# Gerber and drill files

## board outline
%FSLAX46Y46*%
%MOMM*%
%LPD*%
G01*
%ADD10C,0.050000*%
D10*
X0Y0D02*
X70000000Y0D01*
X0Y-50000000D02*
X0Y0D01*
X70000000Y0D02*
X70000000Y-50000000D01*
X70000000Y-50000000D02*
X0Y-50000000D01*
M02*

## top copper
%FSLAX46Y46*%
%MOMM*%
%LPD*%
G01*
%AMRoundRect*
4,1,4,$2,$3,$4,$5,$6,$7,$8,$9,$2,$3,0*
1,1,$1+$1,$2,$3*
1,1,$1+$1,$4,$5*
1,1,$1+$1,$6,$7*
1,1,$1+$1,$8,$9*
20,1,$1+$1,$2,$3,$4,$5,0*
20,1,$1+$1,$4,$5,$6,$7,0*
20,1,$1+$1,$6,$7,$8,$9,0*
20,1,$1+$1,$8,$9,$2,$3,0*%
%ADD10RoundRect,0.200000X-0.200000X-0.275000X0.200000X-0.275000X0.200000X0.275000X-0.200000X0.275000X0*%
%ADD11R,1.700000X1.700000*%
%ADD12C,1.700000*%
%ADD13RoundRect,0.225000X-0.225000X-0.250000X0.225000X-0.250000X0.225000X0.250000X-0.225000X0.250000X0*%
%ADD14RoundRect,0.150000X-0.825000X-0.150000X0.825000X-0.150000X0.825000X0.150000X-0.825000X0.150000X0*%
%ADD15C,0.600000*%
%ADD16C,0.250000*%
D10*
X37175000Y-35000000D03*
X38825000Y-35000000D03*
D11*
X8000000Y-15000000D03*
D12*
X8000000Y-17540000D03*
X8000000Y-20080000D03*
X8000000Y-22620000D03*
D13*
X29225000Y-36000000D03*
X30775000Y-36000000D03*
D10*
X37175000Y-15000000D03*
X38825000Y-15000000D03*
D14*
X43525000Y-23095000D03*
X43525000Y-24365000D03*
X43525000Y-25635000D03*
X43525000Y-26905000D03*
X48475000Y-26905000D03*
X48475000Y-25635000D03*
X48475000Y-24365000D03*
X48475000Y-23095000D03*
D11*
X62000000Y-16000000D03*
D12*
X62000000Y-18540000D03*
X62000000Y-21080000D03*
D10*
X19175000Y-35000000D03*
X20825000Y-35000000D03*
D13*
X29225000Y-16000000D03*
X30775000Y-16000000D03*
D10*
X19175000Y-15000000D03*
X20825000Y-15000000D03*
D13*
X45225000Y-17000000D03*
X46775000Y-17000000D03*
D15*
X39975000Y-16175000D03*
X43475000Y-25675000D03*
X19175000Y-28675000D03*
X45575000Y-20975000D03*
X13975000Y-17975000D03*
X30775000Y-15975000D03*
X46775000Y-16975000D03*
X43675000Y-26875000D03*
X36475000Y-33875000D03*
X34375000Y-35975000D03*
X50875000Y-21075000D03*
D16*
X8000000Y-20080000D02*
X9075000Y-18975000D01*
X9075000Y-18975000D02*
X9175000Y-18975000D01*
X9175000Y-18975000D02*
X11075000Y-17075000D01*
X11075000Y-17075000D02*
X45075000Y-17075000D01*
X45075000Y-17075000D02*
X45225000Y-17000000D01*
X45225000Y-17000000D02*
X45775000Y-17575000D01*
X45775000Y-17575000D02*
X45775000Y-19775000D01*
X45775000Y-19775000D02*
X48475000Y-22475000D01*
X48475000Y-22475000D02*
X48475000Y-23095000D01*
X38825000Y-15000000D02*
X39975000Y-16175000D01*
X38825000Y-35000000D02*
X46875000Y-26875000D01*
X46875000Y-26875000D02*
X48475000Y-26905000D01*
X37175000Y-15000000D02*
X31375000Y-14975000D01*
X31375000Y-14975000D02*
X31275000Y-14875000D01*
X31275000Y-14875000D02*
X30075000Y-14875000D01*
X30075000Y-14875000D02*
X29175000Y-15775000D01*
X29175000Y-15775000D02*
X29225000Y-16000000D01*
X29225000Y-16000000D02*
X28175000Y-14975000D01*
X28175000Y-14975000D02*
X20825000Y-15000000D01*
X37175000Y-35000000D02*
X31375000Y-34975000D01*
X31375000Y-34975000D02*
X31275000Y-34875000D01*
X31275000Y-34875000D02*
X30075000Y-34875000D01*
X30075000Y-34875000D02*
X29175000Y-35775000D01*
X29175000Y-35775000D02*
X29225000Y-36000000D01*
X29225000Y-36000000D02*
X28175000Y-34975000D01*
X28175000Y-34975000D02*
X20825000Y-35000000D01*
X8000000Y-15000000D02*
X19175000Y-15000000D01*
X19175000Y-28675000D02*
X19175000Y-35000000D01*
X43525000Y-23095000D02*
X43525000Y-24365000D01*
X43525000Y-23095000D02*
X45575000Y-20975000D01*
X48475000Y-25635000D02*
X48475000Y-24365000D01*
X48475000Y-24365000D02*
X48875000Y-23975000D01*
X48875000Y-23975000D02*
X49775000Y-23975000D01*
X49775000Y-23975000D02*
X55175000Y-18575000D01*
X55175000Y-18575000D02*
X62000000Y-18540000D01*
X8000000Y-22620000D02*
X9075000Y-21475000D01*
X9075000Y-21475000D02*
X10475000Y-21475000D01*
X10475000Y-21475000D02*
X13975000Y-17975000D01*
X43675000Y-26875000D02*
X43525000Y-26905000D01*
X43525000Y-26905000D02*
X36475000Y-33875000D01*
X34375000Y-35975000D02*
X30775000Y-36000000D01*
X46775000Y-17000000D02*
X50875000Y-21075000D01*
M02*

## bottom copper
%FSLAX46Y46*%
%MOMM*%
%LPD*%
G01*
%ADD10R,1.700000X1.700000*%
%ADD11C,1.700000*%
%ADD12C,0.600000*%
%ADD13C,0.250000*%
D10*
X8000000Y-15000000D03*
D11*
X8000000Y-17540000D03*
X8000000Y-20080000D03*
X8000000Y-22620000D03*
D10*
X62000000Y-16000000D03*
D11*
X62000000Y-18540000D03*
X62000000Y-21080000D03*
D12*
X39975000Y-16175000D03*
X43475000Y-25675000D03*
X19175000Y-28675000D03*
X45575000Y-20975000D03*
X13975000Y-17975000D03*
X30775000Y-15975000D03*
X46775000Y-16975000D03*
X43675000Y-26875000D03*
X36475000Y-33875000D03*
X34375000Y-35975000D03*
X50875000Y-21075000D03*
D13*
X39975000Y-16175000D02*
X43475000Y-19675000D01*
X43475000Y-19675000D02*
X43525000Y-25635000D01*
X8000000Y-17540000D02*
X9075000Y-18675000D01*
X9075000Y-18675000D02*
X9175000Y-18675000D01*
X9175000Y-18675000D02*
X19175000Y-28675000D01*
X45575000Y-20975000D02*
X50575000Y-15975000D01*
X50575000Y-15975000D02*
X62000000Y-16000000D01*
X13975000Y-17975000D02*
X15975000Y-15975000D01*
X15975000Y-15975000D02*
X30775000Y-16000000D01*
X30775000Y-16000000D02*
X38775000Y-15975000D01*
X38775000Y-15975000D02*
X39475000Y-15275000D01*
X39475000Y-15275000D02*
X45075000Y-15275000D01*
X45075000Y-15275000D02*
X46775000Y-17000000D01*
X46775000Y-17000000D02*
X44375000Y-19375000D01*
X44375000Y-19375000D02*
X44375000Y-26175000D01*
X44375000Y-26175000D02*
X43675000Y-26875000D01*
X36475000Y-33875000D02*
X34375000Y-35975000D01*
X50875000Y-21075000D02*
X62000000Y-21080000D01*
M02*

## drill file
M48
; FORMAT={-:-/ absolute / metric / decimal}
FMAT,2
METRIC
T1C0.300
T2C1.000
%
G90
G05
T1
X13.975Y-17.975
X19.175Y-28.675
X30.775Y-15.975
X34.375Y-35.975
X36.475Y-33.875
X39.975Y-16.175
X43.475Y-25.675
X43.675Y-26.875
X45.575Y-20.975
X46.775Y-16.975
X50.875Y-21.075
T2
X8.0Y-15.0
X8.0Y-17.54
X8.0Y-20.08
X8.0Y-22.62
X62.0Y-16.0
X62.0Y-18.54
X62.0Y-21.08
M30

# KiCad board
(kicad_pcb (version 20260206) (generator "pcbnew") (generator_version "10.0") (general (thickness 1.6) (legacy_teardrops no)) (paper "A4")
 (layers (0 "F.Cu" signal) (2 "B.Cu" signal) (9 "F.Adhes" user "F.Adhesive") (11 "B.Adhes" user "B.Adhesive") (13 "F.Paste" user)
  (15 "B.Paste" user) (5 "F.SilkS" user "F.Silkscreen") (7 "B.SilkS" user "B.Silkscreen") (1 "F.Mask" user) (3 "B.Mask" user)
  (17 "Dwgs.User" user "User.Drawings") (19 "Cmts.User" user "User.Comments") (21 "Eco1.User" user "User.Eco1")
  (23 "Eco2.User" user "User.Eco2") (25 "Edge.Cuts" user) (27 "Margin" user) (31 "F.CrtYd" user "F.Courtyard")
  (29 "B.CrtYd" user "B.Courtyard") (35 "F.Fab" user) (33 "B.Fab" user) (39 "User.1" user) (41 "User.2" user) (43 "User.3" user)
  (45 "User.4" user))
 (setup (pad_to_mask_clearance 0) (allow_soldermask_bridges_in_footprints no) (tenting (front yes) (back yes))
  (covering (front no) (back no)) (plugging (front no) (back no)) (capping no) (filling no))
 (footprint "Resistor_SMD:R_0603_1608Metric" (layer "F.Cu") (at 38 35)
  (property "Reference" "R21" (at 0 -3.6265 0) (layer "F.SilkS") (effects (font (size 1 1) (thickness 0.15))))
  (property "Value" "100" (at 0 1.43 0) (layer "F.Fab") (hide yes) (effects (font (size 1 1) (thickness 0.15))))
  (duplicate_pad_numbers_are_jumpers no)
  (pad "1" smd roundrect (at -0.825 0) (size 0.8 0.95) (layers "F.Cu" "F.Mask" "F.Paste") (roundrect_rratio 0.25) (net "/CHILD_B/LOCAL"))
  (pad "2" smd roundrect (at 0.825 0) (size 0.8 0.95) (layers "F.Cu" "F.Mask" "F.Paste") (roundrect_rratio 0.25) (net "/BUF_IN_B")))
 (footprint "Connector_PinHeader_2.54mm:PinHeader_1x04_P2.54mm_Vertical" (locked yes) (layer "F.Cu") (at 8 15)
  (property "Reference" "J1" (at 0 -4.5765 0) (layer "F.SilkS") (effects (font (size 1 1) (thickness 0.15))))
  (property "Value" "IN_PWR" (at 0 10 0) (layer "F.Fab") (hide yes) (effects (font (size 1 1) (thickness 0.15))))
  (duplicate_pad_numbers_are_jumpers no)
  (pad "1" thru_hole rect (at 0 0) (size 1.7 1.7) (drill 1) (layers "*.Cu" "*.Mask") (remove_unused_layers no) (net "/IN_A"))
  (pad "2" thru_hole circle (at 0 2.54) (size 1.7 1.7) (drill 1) (layers "*.Cu" "*.Mask") (remove_unused_layers no) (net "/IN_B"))
  (pad "3" thru_hole circle (at 0 5.08) (size 1.7 1.7) (drill 1) (layers "*.Cu" "*.Mask") (remove_unused_layers no) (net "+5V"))
  (pad "4" thru_hole circle (at 0 7.62) (size 1.7 1.7) (drill 1) (layers "*.Cu" "*.Mask") (remove_unused_layers no) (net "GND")))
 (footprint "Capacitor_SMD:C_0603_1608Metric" (layer "F.Cu") (at 30 36)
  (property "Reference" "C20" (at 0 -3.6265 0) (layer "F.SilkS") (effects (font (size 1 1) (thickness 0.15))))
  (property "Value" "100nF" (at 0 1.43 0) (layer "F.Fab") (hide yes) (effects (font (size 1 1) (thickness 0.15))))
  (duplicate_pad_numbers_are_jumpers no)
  (pad "1" smd roundrect (at -0.775 0) (size 0.9 0.95) (layers "F.Cu" "F.Mask" "F.Paste") (roundrect_rratio 0.25) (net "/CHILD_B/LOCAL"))
  (pad "2" smd roundrect (at 0.775 0) (size 0.9 0.95) (layers "F.Cu" "F.Mask" "F.Paste") (roundrect_rratio 0.25) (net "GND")))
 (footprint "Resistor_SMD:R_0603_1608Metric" (layer "F.Cu") (at 38 15)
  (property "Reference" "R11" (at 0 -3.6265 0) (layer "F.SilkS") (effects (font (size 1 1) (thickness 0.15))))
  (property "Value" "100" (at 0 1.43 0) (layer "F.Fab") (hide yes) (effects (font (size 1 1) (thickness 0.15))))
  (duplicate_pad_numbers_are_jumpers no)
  (pad "1" smd roundrect (at -0.825 0) (size 0.8 0.95) (layers "F.Cu" "F.Mask" "F.Paste") (roundrect_rratio 0.25) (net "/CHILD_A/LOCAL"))
  (pad "2" smd roundrect (at 0.825 0) (size 0.8 0.95) (layers "F.Cu" "F.Mask" "F.Paste") (roundrect_rratio 0.25) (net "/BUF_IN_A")))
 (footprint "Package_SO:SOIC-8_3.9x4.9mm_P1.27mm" (layer "F.Cu") (at 46 25)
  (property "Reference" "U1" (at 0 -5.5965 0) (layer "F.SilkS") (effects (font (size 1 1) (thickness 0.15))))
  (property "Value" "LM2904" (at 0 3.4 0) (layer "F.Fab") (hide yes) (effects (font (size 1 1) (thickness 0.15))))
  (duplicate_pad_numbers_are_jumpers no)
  (pad "1" smd roundrect (at -2.475 -1.905) (size 1.95 0.6) (layers "F.Cu" "F.Mask" "F.Paste") (roundrect_rratio 0.25) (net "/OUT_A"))
  (pad "2" smd roundrect (at -2.475 -0.635) (size 1.95 0.6) (layers "F.Cu" "F.Mask" "F.Paste") (roundrect_rratio 0.25) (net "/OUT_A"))
  (pad "3" smd roundrect (at -2.475 0.635) (size 1.95 0.6) (layers "F.Cu" "F.Mask" "F.Paste") (roundrect_rratio 0.25) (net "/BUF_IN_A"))
  (pad "4" smd roundrect (at -2.475 1.905) (size 1.95 0.6) (layers "F.Cu" "F.Mask" "F.Paste") (roundrect_rratio 0.25) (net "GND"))
  (pad "5" smd roundrect (at 2.475 1.905) (size 1.95 0.6) (layers "F.Cu" "F.Mask" "F.Paste") (roundrect_rratio 0.25) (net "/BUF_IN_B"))
  (pad "6" smd roundrect (at 2.475 0.635) (size 1.95 0.6) (layers "F.Cu" "F.Mask" "F.Paste") (roundrect_rratio 0.25) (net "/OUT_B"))
  (pad "7" smd roundrect (at 2.475 -0.635) (size 1.95 0.6) (layers "F.Cu" "F.Mask" "F.Paste") (roundrect_rratio 0.25) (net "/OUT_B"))
  (pad "8" smd roundrect (at 2.475 -1.905) (size 1.95 0.6) (layers "F.Cu" "F.Mask" "F.Paste") (roundrect_rratio 0.25) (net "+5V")))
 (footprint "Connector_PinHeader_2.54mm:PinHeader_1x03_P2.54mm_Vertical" (layer "F.Cu") (at 62 16)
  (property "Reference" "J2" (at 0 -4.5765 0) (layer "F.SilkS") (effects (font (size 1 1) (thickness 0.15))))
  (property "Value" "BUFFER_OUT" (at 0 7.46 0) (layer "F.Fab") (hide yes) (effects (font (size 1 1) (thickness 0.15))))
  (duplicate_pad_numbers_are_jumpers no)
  (pad "1" thru_hole rect (at 0 0) (size 1.7 1.7) (drill 1) (layers "*.Cu" "*.Mask") (remove_unused_layers no) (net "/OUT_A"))
  (pad "2" thru_hole circle (at 0 2.54) (size 1.7 1.7) (drill 1) (layers "*.Cu" "*.Mask") (remove_unused_layers no) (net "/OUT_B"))
  (pad "3" thru_hole circle (at 0 5.08) (size 1.7 1.7) (drill 1) (layers "*.Cu" "*.Mask") (remove_unused_layers no) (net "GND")))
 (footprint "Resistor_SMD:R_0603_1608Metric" (layer "F.Cu") (at 20 35)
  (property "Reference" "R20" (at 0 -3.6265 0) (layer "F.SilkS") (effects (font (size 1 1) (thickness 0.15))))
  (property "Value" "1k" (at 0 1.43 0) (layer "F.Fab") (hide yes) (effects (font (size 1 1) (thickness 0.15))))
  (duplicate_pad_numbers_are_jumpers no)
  (pad "1" smd roundrect (at -0.825 0) (size 0.8 0.95) (layers "F.Cu" "F.Mask" "F.Paste") (roundrect_rratio 0.25) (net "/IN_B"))
  (pad "2" smd roundrect (at 0.825 0) (size 0.8 0.95) (layers "F.Cu" "F.Mask" "F.Paste") (roundrect_rratio 0.25) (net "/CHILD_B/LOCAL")))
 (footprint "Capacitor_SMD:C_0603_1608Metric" (layer "F.Cu") (at 30 16)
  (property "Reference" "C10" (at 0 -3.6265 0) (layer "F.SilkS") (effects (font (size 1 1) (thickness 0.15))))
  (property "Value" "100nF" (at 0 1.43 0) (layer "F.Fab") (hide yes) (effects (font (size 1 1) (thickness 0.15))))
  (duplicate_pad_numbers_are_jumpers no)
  (pad "1" smd roundrect (at -0.775 0) (size 0.9 0.95) (layers "F.Cu" "F.Mask" "F.Paste") (roundrect_rratio 0.25) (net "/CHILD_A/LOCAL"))
  (pad "2" smd roundrect (at 0.775 0) (size 0.9 0.95) (layers "F.Cu" "F.Mask" "F.Paste") (roundrect_rratio 0.25) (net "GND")))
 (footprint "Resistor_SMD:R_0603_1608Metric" (layer "F.Cu") (at 20 15)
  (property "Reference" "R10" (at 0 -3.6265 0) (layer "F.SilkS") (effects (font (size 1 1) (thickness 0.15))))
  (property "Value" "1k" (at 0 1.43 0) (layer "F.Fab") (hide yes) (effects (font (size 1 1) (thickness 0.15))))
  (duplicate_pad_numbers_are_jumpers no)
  (pad "1" smd roundrect (at -0.825 0) (size 0.8 0.95) (layers "F.Cu" "F.Mask" "F.Paste") (roundrect_rratio 0.25) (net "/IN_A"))
  (pad "2" smd roundrect (at 0.825 0) (size 0.8 0.95) (layers "F.Cu" "F.Mask" "F.Paste") (roundrect_rratio 0.25) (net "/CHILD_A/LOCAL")))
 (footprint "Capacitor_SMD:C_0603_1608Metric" (layer "F.Cu") (at 46 17)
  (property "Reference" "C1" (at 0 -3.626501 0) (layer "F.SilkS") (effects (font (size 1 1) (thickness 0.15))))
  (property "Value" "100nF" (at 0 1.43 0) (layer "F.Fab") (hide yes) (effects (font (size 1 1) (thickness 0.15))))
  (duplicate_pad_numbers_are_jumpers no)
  (pad "1" smd roundrect (at -0.775 0) (size 0.9 0.95) (layers "F.Cu" "F.Mask" "F.Paste") (roundrect_rratio 0.25) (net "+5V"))
  (pad "2" smd roundrect (at 0.775 0) (size 0.9 0.95) (layers "F.Cu" "F.Mask" "F.Paste") (roundrect_rratio 0.25) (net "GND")))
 (gr_line (start 0 0) (end 70 0) (stroke (width 0.05) (type default)) (layer "Edge.Cuts"))
 (gr_line (start 0 50) (end 0 0) (stroke (width 0.05) (type default)) (layer "Edge.Cuts"))
 (gr_line (start 70 0) (end 70 50) (stroke (width 0.05) (type default)) (layer "Edge.Cuts"))
 (gr_line (start 70 50) (end 0 50) (stroke (width 0.05) (type default)) (layer "Edge.Cuts"))
 (segment (start 8 20.08) (end 9.075 18.975) (width 0.25) (layer "F.Cu") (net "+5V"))
 (segment (start 9.075 18.975) (end 9.175 18.975) (width 0.25) (layer "F.Cu") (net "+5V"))
 (segment (start 9.175 18.975) (end 11.075 17.075) (width 0.25) (layer "F.Cu") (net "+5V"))
 (segment (start 11.075 17.075) (end 45.075 17.075) (width 0.25) (layer "F.Cu") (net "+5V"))
 (segment (start 45.075 17.075) (end 45.225 17) (width 0.25) (layer "F.Cu") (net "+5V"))
 (segment (start 45.225 17) (end 45.775 17.575) (width 0.25) (layer "F.Cu") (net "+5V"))
 (segment (start 45.775 17.575) (end 45.775 19.775) (width 0.25) (layer "F.Cu") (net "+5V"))
 (segment (start 45.775 19.775) (end 48.475 22.475) (width 0.25) (layer "F.Cu") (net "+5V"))
 (segment (start 48.475 22.475) (end 48.475 23.095) (width 0.25) (layer "F.Cu") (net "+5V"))
 (segment (start 38.825 15) (end 39.975 16.175) (width 0.25) (layer "F.Cu") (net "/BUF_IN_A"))
 (via (at 39.975 16.175) (size 0.6) (drill 0.3) (layers "F.Cu" "B.Cu") (capping no) (covering (front no) (back no))
  (plugging (front no) (back no)) (filling no) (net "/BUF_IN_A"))
 (segment (start 39.975 16.175) (end 43.475 19.675) (width 0.25) (layer "B.Cu") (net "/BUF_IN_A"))
 (segment (start 43.475 19.675) (end 43.525 25.635) (width 0.25) (layer "B.Cu") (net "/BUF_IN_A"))
 (via (at 43.475 25.675) (size 0.6) (drill 0.3) (layers "F.Cu" "B.Cu") (capping no) (covering (front no) (back no))
  (plugging (front no) (back no)) (filling no) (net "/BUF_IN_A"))
 (segment (start 38.825 35) (end 46.875 26.875) (width 0.25) (layer "F.Cu") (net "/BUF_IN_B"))
 (segment (start 46.875 26.875) (end 48.475 26.905) (width 0.25) (layer "F.Cu") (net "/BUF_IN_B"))
 (segment (start 37.175 15) (end 31.375 14.975) (width 0.25) (layer "F.Cu") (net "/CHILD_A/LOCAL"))
 (segment (start 31.375 14.975) (end 31.275 14.875) (width 0.25) (layer "F.Cu") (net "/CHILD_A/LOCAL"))
 (segment (start 31.275 14.875) (end 30.075 14.875) (width 0.25) (layer "F.Cu") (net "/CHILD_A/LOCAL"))
 (segment (start 30.075 14.875) (end 29.175 15.775) (width 0.25) (layer "F.Cu") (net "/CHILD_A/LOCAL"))
 (segment (start 29.175 15.775) (end 29.225 16) (width 0.25) (layer "F.Cu") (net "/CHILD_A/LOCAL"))
 (segment (start 29.225 16) (end 28.175 14.975) (width 0.25) (layer "F.Cu") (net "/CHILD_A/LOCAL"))
 (segment (start 28.175 14.975) (end 20.825 15) (width 0.25) (layer "F.Cu") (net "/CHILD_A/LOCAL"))
 (segment (start 37.175 35) (end 31.375 34.975) (width 0.25) (layer "F.Cu") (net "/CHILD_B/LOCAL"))
 (segment (start 31.375 34.975) (end 31.275 34.875) (width 0.25) (layer "F.Cu") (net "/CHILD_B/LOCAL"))
 (segment (start 31.275 34.875) (end 30.075 34.875) (width 0.25) (layer "F.Cu") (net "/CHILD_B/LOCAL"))
 (segment (start 30.075 34.875) (end 29.175 35.775) (width 0.25) (layer "F.Cu") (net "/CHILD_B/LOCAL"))
 (segment (start 29.175 35.775) (end 29.225 36) (width 0.25) (layer "F.Cu") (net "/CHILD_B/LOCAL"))
 (segment (start 29.225 36) (end 28.175 34.975) (width 0.25) (layer "F.Cu") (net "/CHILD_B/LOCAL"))
 (segment (start 28.175 34.975) (end 20.825 35) (width 0.25) (layer "F.Cu") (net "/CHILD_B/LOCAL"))
 (segment (start 8 15) (end 19.175 15) (width 0.25) (layer "F.Cu") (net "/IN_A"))
 (segment (start 8 17.54) (end 9.075 18.675) (width 0.25) (layer "B.Cu") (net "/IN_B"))
 (segment (start 9.075 18.675) (end 9.175 18.675) (width 0.25) (layer "B.Cu") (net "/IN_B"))
 (segment (start 9.175 18.675) (end 19.175 28.675) (width 0.25) (layer "B.Cu") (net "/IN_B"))
 (via (at 19.175 28.675) (size 0.6) (drill 0.3) (layers "F.Cu" "B.Cu") (capping no) (covering (front no) (back no))
  (plugging (front no) (back no)) (filling no) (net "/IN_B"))
 (segment (start 19.175 28.675) (end 19.175 35) (width 0.25) (layer "F.Cu") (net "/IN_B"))
 (segment (start 43.525 23.095) (end 43.525 24.365) (width 0.25) (layer "F.Cu") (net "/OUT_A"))
 (segment (start 43.525 23.095) (end 45.575 20.975) (width 0.25) (layer "F.Cu") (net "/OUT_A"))
 (via (at 45.575 20.975) (size 0.6) (drill 0.3) (layers "F.Cu" "B.Cu") (capping no) (covering (front no) (back no))
  (plugging (front no) (back no)) (filling no) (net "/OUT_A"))
 (segment (start 45.575 20.975) (end 50.575 15.975) (width 0.25) (layer "B.Cu") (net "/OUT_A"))
 (segment (start 50.575 15.975) (end 62 16) (width 0.25) (layer "B.Cu") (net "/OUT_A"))
 (segment (start 48.475 25.635) (end 48.475 24.365) (width 0.25) (layer "F.Cu") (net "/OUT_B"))
 (segment (start 48.475 24.365) (end 48.875 23.975) (width 0.25) (layer "F.Cu") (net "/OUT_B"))
 (segment (start 48.875 23.975) (end 49.775 23.975) (width 0.25) (layer "F.Cu") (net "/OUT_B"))
 (segment (start 49.775 23.975) (end 55.175 18.575) (width 0.25) (layer "F.Cu") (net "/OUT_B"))
 (segment (start 55.175 18.575) (end 62 18.54) (width 0.25) (layer "F.Cu") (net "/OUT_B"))
 (segment (start 8 22.62) (end 9.075 21.475) (width 0.25) (layer "F.Cu") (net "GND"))
 (segment (start 9.075 21.475) (end 10.475 21.475) (width 0.25) (layer "F.Cu") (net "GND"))
 (segment (start 10.475 21.475) (end 13.975 17.975) (width 0.25) (layer "F.Cu") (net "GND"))
 (via (at 13.975 17.975) (size 0.6) (drill 0.3) (layers "F.Cu" "B.Cu") (capping no) (covering (front no) (back no))
  (plugging (front no) (back no)) (filling no) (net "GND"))
 (segment (start 13.975 17.975) (end 15.975 15.975) (width 0.25) (layer "B.Cu") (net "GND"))
 (segment (start 15.975 15.975) (end 30.775 16) (width 0.25) (layer "B.Cu") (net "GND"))
 (via (at 30.775 15.975) (size 0.6) (drill 0.3) (layers "F.Cu" "B.Cu") (capping no) (covering (front no) (back no))
  (plugging (front no) (back no)) (filling no) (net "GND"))
 (segment (start 30.775 16) (end 38.775 15.975) (width 0.25) (layer "B.Cu") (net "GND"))
 (segment (start 38.775 15.975) (end 39.475 15.275) (width 0.25) (layer "B.Cu") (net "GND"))
 (segment (start 39.475 15.275) (end 45.075 15.275) (width 0.25) (layer "B.Cu") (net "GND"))
 (segment (start 45.075 15.275) (end 46.775 17) (width 0.25) (layer "B.Cu") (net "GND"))
 (via (at 46.775 16.975) (size 0.6) (drill 0.3) (layers "F.Cu" "B.Cu") (capping no) (covering (front no) (back no))
  (plugging (front no) (back no)) (filling no) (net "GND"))
 (segment (start 46.775 17) (end 44.375 19.375) (width 0.25) (layer "B.Cu") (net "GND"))
 (segment (start 44.375 19.375) (end 44.375 26.175) (width 0.25) (layer "B.Cu") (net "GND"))
 (segment (start 44.375 26.175) (end 43.675 26.875) (width 0.25) (layer "B.Cu") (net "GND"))
 (via (at 43.675 26.875) (size 0.6) (drill 0.3) (layers "F.Cu" "B.Cu") (capping no) (covering (front no) (back no))
  (plugging (front no) (back no)) (filling no) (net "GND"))
 (segment (start 43.675 26.875) (end 43.525 26.905) (width 0.25) (layer "F.Cu") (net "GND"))
 (segment (start 43.525 26.905) (end 36.475 33.875) (width 0.25) (layer "F.Cu") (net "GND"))
 (via (at 36.475 33.875) (size 0.6) (drill 0.3) (layers "F.Cu" "B.Cu") (capping no) (covering (front no) (back no))
  (plugging (front no) (back no)) (filling no) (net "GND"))
 (segment (start 36.475 33.875) (end 34.375 35.975) (width 0.25) (layer "B.Cu") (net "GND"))
 (via (at 34.375 35.975) (size 0.6) (drill 0.3) (layers "F.Cu" "B.Cu") (capping no) (covering (front no) (back no))
  (plugging (front no) (back no)) (filling no) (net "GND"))
 (segment (start 34.375 35.975) (end 30.775 36) (width 0.25) (layer "F.Cu") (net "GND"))
 (segment (start 46.775 17) (end 50.875 21.075) (width 0.25) (layer "F.Cu") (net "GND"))
 (via (at 50.875 21.075) (size 0.6) (drill 0.3) (layers "F.Cu" "B.Cu") (capping no) (covering (front no) (back no))
  (plugging (front no) (back no)) (filling no) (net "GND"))
 (segment (start 50.875 21.075) (end 62 21.08) (width 0.25) (layer "B.Cu") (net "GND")))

